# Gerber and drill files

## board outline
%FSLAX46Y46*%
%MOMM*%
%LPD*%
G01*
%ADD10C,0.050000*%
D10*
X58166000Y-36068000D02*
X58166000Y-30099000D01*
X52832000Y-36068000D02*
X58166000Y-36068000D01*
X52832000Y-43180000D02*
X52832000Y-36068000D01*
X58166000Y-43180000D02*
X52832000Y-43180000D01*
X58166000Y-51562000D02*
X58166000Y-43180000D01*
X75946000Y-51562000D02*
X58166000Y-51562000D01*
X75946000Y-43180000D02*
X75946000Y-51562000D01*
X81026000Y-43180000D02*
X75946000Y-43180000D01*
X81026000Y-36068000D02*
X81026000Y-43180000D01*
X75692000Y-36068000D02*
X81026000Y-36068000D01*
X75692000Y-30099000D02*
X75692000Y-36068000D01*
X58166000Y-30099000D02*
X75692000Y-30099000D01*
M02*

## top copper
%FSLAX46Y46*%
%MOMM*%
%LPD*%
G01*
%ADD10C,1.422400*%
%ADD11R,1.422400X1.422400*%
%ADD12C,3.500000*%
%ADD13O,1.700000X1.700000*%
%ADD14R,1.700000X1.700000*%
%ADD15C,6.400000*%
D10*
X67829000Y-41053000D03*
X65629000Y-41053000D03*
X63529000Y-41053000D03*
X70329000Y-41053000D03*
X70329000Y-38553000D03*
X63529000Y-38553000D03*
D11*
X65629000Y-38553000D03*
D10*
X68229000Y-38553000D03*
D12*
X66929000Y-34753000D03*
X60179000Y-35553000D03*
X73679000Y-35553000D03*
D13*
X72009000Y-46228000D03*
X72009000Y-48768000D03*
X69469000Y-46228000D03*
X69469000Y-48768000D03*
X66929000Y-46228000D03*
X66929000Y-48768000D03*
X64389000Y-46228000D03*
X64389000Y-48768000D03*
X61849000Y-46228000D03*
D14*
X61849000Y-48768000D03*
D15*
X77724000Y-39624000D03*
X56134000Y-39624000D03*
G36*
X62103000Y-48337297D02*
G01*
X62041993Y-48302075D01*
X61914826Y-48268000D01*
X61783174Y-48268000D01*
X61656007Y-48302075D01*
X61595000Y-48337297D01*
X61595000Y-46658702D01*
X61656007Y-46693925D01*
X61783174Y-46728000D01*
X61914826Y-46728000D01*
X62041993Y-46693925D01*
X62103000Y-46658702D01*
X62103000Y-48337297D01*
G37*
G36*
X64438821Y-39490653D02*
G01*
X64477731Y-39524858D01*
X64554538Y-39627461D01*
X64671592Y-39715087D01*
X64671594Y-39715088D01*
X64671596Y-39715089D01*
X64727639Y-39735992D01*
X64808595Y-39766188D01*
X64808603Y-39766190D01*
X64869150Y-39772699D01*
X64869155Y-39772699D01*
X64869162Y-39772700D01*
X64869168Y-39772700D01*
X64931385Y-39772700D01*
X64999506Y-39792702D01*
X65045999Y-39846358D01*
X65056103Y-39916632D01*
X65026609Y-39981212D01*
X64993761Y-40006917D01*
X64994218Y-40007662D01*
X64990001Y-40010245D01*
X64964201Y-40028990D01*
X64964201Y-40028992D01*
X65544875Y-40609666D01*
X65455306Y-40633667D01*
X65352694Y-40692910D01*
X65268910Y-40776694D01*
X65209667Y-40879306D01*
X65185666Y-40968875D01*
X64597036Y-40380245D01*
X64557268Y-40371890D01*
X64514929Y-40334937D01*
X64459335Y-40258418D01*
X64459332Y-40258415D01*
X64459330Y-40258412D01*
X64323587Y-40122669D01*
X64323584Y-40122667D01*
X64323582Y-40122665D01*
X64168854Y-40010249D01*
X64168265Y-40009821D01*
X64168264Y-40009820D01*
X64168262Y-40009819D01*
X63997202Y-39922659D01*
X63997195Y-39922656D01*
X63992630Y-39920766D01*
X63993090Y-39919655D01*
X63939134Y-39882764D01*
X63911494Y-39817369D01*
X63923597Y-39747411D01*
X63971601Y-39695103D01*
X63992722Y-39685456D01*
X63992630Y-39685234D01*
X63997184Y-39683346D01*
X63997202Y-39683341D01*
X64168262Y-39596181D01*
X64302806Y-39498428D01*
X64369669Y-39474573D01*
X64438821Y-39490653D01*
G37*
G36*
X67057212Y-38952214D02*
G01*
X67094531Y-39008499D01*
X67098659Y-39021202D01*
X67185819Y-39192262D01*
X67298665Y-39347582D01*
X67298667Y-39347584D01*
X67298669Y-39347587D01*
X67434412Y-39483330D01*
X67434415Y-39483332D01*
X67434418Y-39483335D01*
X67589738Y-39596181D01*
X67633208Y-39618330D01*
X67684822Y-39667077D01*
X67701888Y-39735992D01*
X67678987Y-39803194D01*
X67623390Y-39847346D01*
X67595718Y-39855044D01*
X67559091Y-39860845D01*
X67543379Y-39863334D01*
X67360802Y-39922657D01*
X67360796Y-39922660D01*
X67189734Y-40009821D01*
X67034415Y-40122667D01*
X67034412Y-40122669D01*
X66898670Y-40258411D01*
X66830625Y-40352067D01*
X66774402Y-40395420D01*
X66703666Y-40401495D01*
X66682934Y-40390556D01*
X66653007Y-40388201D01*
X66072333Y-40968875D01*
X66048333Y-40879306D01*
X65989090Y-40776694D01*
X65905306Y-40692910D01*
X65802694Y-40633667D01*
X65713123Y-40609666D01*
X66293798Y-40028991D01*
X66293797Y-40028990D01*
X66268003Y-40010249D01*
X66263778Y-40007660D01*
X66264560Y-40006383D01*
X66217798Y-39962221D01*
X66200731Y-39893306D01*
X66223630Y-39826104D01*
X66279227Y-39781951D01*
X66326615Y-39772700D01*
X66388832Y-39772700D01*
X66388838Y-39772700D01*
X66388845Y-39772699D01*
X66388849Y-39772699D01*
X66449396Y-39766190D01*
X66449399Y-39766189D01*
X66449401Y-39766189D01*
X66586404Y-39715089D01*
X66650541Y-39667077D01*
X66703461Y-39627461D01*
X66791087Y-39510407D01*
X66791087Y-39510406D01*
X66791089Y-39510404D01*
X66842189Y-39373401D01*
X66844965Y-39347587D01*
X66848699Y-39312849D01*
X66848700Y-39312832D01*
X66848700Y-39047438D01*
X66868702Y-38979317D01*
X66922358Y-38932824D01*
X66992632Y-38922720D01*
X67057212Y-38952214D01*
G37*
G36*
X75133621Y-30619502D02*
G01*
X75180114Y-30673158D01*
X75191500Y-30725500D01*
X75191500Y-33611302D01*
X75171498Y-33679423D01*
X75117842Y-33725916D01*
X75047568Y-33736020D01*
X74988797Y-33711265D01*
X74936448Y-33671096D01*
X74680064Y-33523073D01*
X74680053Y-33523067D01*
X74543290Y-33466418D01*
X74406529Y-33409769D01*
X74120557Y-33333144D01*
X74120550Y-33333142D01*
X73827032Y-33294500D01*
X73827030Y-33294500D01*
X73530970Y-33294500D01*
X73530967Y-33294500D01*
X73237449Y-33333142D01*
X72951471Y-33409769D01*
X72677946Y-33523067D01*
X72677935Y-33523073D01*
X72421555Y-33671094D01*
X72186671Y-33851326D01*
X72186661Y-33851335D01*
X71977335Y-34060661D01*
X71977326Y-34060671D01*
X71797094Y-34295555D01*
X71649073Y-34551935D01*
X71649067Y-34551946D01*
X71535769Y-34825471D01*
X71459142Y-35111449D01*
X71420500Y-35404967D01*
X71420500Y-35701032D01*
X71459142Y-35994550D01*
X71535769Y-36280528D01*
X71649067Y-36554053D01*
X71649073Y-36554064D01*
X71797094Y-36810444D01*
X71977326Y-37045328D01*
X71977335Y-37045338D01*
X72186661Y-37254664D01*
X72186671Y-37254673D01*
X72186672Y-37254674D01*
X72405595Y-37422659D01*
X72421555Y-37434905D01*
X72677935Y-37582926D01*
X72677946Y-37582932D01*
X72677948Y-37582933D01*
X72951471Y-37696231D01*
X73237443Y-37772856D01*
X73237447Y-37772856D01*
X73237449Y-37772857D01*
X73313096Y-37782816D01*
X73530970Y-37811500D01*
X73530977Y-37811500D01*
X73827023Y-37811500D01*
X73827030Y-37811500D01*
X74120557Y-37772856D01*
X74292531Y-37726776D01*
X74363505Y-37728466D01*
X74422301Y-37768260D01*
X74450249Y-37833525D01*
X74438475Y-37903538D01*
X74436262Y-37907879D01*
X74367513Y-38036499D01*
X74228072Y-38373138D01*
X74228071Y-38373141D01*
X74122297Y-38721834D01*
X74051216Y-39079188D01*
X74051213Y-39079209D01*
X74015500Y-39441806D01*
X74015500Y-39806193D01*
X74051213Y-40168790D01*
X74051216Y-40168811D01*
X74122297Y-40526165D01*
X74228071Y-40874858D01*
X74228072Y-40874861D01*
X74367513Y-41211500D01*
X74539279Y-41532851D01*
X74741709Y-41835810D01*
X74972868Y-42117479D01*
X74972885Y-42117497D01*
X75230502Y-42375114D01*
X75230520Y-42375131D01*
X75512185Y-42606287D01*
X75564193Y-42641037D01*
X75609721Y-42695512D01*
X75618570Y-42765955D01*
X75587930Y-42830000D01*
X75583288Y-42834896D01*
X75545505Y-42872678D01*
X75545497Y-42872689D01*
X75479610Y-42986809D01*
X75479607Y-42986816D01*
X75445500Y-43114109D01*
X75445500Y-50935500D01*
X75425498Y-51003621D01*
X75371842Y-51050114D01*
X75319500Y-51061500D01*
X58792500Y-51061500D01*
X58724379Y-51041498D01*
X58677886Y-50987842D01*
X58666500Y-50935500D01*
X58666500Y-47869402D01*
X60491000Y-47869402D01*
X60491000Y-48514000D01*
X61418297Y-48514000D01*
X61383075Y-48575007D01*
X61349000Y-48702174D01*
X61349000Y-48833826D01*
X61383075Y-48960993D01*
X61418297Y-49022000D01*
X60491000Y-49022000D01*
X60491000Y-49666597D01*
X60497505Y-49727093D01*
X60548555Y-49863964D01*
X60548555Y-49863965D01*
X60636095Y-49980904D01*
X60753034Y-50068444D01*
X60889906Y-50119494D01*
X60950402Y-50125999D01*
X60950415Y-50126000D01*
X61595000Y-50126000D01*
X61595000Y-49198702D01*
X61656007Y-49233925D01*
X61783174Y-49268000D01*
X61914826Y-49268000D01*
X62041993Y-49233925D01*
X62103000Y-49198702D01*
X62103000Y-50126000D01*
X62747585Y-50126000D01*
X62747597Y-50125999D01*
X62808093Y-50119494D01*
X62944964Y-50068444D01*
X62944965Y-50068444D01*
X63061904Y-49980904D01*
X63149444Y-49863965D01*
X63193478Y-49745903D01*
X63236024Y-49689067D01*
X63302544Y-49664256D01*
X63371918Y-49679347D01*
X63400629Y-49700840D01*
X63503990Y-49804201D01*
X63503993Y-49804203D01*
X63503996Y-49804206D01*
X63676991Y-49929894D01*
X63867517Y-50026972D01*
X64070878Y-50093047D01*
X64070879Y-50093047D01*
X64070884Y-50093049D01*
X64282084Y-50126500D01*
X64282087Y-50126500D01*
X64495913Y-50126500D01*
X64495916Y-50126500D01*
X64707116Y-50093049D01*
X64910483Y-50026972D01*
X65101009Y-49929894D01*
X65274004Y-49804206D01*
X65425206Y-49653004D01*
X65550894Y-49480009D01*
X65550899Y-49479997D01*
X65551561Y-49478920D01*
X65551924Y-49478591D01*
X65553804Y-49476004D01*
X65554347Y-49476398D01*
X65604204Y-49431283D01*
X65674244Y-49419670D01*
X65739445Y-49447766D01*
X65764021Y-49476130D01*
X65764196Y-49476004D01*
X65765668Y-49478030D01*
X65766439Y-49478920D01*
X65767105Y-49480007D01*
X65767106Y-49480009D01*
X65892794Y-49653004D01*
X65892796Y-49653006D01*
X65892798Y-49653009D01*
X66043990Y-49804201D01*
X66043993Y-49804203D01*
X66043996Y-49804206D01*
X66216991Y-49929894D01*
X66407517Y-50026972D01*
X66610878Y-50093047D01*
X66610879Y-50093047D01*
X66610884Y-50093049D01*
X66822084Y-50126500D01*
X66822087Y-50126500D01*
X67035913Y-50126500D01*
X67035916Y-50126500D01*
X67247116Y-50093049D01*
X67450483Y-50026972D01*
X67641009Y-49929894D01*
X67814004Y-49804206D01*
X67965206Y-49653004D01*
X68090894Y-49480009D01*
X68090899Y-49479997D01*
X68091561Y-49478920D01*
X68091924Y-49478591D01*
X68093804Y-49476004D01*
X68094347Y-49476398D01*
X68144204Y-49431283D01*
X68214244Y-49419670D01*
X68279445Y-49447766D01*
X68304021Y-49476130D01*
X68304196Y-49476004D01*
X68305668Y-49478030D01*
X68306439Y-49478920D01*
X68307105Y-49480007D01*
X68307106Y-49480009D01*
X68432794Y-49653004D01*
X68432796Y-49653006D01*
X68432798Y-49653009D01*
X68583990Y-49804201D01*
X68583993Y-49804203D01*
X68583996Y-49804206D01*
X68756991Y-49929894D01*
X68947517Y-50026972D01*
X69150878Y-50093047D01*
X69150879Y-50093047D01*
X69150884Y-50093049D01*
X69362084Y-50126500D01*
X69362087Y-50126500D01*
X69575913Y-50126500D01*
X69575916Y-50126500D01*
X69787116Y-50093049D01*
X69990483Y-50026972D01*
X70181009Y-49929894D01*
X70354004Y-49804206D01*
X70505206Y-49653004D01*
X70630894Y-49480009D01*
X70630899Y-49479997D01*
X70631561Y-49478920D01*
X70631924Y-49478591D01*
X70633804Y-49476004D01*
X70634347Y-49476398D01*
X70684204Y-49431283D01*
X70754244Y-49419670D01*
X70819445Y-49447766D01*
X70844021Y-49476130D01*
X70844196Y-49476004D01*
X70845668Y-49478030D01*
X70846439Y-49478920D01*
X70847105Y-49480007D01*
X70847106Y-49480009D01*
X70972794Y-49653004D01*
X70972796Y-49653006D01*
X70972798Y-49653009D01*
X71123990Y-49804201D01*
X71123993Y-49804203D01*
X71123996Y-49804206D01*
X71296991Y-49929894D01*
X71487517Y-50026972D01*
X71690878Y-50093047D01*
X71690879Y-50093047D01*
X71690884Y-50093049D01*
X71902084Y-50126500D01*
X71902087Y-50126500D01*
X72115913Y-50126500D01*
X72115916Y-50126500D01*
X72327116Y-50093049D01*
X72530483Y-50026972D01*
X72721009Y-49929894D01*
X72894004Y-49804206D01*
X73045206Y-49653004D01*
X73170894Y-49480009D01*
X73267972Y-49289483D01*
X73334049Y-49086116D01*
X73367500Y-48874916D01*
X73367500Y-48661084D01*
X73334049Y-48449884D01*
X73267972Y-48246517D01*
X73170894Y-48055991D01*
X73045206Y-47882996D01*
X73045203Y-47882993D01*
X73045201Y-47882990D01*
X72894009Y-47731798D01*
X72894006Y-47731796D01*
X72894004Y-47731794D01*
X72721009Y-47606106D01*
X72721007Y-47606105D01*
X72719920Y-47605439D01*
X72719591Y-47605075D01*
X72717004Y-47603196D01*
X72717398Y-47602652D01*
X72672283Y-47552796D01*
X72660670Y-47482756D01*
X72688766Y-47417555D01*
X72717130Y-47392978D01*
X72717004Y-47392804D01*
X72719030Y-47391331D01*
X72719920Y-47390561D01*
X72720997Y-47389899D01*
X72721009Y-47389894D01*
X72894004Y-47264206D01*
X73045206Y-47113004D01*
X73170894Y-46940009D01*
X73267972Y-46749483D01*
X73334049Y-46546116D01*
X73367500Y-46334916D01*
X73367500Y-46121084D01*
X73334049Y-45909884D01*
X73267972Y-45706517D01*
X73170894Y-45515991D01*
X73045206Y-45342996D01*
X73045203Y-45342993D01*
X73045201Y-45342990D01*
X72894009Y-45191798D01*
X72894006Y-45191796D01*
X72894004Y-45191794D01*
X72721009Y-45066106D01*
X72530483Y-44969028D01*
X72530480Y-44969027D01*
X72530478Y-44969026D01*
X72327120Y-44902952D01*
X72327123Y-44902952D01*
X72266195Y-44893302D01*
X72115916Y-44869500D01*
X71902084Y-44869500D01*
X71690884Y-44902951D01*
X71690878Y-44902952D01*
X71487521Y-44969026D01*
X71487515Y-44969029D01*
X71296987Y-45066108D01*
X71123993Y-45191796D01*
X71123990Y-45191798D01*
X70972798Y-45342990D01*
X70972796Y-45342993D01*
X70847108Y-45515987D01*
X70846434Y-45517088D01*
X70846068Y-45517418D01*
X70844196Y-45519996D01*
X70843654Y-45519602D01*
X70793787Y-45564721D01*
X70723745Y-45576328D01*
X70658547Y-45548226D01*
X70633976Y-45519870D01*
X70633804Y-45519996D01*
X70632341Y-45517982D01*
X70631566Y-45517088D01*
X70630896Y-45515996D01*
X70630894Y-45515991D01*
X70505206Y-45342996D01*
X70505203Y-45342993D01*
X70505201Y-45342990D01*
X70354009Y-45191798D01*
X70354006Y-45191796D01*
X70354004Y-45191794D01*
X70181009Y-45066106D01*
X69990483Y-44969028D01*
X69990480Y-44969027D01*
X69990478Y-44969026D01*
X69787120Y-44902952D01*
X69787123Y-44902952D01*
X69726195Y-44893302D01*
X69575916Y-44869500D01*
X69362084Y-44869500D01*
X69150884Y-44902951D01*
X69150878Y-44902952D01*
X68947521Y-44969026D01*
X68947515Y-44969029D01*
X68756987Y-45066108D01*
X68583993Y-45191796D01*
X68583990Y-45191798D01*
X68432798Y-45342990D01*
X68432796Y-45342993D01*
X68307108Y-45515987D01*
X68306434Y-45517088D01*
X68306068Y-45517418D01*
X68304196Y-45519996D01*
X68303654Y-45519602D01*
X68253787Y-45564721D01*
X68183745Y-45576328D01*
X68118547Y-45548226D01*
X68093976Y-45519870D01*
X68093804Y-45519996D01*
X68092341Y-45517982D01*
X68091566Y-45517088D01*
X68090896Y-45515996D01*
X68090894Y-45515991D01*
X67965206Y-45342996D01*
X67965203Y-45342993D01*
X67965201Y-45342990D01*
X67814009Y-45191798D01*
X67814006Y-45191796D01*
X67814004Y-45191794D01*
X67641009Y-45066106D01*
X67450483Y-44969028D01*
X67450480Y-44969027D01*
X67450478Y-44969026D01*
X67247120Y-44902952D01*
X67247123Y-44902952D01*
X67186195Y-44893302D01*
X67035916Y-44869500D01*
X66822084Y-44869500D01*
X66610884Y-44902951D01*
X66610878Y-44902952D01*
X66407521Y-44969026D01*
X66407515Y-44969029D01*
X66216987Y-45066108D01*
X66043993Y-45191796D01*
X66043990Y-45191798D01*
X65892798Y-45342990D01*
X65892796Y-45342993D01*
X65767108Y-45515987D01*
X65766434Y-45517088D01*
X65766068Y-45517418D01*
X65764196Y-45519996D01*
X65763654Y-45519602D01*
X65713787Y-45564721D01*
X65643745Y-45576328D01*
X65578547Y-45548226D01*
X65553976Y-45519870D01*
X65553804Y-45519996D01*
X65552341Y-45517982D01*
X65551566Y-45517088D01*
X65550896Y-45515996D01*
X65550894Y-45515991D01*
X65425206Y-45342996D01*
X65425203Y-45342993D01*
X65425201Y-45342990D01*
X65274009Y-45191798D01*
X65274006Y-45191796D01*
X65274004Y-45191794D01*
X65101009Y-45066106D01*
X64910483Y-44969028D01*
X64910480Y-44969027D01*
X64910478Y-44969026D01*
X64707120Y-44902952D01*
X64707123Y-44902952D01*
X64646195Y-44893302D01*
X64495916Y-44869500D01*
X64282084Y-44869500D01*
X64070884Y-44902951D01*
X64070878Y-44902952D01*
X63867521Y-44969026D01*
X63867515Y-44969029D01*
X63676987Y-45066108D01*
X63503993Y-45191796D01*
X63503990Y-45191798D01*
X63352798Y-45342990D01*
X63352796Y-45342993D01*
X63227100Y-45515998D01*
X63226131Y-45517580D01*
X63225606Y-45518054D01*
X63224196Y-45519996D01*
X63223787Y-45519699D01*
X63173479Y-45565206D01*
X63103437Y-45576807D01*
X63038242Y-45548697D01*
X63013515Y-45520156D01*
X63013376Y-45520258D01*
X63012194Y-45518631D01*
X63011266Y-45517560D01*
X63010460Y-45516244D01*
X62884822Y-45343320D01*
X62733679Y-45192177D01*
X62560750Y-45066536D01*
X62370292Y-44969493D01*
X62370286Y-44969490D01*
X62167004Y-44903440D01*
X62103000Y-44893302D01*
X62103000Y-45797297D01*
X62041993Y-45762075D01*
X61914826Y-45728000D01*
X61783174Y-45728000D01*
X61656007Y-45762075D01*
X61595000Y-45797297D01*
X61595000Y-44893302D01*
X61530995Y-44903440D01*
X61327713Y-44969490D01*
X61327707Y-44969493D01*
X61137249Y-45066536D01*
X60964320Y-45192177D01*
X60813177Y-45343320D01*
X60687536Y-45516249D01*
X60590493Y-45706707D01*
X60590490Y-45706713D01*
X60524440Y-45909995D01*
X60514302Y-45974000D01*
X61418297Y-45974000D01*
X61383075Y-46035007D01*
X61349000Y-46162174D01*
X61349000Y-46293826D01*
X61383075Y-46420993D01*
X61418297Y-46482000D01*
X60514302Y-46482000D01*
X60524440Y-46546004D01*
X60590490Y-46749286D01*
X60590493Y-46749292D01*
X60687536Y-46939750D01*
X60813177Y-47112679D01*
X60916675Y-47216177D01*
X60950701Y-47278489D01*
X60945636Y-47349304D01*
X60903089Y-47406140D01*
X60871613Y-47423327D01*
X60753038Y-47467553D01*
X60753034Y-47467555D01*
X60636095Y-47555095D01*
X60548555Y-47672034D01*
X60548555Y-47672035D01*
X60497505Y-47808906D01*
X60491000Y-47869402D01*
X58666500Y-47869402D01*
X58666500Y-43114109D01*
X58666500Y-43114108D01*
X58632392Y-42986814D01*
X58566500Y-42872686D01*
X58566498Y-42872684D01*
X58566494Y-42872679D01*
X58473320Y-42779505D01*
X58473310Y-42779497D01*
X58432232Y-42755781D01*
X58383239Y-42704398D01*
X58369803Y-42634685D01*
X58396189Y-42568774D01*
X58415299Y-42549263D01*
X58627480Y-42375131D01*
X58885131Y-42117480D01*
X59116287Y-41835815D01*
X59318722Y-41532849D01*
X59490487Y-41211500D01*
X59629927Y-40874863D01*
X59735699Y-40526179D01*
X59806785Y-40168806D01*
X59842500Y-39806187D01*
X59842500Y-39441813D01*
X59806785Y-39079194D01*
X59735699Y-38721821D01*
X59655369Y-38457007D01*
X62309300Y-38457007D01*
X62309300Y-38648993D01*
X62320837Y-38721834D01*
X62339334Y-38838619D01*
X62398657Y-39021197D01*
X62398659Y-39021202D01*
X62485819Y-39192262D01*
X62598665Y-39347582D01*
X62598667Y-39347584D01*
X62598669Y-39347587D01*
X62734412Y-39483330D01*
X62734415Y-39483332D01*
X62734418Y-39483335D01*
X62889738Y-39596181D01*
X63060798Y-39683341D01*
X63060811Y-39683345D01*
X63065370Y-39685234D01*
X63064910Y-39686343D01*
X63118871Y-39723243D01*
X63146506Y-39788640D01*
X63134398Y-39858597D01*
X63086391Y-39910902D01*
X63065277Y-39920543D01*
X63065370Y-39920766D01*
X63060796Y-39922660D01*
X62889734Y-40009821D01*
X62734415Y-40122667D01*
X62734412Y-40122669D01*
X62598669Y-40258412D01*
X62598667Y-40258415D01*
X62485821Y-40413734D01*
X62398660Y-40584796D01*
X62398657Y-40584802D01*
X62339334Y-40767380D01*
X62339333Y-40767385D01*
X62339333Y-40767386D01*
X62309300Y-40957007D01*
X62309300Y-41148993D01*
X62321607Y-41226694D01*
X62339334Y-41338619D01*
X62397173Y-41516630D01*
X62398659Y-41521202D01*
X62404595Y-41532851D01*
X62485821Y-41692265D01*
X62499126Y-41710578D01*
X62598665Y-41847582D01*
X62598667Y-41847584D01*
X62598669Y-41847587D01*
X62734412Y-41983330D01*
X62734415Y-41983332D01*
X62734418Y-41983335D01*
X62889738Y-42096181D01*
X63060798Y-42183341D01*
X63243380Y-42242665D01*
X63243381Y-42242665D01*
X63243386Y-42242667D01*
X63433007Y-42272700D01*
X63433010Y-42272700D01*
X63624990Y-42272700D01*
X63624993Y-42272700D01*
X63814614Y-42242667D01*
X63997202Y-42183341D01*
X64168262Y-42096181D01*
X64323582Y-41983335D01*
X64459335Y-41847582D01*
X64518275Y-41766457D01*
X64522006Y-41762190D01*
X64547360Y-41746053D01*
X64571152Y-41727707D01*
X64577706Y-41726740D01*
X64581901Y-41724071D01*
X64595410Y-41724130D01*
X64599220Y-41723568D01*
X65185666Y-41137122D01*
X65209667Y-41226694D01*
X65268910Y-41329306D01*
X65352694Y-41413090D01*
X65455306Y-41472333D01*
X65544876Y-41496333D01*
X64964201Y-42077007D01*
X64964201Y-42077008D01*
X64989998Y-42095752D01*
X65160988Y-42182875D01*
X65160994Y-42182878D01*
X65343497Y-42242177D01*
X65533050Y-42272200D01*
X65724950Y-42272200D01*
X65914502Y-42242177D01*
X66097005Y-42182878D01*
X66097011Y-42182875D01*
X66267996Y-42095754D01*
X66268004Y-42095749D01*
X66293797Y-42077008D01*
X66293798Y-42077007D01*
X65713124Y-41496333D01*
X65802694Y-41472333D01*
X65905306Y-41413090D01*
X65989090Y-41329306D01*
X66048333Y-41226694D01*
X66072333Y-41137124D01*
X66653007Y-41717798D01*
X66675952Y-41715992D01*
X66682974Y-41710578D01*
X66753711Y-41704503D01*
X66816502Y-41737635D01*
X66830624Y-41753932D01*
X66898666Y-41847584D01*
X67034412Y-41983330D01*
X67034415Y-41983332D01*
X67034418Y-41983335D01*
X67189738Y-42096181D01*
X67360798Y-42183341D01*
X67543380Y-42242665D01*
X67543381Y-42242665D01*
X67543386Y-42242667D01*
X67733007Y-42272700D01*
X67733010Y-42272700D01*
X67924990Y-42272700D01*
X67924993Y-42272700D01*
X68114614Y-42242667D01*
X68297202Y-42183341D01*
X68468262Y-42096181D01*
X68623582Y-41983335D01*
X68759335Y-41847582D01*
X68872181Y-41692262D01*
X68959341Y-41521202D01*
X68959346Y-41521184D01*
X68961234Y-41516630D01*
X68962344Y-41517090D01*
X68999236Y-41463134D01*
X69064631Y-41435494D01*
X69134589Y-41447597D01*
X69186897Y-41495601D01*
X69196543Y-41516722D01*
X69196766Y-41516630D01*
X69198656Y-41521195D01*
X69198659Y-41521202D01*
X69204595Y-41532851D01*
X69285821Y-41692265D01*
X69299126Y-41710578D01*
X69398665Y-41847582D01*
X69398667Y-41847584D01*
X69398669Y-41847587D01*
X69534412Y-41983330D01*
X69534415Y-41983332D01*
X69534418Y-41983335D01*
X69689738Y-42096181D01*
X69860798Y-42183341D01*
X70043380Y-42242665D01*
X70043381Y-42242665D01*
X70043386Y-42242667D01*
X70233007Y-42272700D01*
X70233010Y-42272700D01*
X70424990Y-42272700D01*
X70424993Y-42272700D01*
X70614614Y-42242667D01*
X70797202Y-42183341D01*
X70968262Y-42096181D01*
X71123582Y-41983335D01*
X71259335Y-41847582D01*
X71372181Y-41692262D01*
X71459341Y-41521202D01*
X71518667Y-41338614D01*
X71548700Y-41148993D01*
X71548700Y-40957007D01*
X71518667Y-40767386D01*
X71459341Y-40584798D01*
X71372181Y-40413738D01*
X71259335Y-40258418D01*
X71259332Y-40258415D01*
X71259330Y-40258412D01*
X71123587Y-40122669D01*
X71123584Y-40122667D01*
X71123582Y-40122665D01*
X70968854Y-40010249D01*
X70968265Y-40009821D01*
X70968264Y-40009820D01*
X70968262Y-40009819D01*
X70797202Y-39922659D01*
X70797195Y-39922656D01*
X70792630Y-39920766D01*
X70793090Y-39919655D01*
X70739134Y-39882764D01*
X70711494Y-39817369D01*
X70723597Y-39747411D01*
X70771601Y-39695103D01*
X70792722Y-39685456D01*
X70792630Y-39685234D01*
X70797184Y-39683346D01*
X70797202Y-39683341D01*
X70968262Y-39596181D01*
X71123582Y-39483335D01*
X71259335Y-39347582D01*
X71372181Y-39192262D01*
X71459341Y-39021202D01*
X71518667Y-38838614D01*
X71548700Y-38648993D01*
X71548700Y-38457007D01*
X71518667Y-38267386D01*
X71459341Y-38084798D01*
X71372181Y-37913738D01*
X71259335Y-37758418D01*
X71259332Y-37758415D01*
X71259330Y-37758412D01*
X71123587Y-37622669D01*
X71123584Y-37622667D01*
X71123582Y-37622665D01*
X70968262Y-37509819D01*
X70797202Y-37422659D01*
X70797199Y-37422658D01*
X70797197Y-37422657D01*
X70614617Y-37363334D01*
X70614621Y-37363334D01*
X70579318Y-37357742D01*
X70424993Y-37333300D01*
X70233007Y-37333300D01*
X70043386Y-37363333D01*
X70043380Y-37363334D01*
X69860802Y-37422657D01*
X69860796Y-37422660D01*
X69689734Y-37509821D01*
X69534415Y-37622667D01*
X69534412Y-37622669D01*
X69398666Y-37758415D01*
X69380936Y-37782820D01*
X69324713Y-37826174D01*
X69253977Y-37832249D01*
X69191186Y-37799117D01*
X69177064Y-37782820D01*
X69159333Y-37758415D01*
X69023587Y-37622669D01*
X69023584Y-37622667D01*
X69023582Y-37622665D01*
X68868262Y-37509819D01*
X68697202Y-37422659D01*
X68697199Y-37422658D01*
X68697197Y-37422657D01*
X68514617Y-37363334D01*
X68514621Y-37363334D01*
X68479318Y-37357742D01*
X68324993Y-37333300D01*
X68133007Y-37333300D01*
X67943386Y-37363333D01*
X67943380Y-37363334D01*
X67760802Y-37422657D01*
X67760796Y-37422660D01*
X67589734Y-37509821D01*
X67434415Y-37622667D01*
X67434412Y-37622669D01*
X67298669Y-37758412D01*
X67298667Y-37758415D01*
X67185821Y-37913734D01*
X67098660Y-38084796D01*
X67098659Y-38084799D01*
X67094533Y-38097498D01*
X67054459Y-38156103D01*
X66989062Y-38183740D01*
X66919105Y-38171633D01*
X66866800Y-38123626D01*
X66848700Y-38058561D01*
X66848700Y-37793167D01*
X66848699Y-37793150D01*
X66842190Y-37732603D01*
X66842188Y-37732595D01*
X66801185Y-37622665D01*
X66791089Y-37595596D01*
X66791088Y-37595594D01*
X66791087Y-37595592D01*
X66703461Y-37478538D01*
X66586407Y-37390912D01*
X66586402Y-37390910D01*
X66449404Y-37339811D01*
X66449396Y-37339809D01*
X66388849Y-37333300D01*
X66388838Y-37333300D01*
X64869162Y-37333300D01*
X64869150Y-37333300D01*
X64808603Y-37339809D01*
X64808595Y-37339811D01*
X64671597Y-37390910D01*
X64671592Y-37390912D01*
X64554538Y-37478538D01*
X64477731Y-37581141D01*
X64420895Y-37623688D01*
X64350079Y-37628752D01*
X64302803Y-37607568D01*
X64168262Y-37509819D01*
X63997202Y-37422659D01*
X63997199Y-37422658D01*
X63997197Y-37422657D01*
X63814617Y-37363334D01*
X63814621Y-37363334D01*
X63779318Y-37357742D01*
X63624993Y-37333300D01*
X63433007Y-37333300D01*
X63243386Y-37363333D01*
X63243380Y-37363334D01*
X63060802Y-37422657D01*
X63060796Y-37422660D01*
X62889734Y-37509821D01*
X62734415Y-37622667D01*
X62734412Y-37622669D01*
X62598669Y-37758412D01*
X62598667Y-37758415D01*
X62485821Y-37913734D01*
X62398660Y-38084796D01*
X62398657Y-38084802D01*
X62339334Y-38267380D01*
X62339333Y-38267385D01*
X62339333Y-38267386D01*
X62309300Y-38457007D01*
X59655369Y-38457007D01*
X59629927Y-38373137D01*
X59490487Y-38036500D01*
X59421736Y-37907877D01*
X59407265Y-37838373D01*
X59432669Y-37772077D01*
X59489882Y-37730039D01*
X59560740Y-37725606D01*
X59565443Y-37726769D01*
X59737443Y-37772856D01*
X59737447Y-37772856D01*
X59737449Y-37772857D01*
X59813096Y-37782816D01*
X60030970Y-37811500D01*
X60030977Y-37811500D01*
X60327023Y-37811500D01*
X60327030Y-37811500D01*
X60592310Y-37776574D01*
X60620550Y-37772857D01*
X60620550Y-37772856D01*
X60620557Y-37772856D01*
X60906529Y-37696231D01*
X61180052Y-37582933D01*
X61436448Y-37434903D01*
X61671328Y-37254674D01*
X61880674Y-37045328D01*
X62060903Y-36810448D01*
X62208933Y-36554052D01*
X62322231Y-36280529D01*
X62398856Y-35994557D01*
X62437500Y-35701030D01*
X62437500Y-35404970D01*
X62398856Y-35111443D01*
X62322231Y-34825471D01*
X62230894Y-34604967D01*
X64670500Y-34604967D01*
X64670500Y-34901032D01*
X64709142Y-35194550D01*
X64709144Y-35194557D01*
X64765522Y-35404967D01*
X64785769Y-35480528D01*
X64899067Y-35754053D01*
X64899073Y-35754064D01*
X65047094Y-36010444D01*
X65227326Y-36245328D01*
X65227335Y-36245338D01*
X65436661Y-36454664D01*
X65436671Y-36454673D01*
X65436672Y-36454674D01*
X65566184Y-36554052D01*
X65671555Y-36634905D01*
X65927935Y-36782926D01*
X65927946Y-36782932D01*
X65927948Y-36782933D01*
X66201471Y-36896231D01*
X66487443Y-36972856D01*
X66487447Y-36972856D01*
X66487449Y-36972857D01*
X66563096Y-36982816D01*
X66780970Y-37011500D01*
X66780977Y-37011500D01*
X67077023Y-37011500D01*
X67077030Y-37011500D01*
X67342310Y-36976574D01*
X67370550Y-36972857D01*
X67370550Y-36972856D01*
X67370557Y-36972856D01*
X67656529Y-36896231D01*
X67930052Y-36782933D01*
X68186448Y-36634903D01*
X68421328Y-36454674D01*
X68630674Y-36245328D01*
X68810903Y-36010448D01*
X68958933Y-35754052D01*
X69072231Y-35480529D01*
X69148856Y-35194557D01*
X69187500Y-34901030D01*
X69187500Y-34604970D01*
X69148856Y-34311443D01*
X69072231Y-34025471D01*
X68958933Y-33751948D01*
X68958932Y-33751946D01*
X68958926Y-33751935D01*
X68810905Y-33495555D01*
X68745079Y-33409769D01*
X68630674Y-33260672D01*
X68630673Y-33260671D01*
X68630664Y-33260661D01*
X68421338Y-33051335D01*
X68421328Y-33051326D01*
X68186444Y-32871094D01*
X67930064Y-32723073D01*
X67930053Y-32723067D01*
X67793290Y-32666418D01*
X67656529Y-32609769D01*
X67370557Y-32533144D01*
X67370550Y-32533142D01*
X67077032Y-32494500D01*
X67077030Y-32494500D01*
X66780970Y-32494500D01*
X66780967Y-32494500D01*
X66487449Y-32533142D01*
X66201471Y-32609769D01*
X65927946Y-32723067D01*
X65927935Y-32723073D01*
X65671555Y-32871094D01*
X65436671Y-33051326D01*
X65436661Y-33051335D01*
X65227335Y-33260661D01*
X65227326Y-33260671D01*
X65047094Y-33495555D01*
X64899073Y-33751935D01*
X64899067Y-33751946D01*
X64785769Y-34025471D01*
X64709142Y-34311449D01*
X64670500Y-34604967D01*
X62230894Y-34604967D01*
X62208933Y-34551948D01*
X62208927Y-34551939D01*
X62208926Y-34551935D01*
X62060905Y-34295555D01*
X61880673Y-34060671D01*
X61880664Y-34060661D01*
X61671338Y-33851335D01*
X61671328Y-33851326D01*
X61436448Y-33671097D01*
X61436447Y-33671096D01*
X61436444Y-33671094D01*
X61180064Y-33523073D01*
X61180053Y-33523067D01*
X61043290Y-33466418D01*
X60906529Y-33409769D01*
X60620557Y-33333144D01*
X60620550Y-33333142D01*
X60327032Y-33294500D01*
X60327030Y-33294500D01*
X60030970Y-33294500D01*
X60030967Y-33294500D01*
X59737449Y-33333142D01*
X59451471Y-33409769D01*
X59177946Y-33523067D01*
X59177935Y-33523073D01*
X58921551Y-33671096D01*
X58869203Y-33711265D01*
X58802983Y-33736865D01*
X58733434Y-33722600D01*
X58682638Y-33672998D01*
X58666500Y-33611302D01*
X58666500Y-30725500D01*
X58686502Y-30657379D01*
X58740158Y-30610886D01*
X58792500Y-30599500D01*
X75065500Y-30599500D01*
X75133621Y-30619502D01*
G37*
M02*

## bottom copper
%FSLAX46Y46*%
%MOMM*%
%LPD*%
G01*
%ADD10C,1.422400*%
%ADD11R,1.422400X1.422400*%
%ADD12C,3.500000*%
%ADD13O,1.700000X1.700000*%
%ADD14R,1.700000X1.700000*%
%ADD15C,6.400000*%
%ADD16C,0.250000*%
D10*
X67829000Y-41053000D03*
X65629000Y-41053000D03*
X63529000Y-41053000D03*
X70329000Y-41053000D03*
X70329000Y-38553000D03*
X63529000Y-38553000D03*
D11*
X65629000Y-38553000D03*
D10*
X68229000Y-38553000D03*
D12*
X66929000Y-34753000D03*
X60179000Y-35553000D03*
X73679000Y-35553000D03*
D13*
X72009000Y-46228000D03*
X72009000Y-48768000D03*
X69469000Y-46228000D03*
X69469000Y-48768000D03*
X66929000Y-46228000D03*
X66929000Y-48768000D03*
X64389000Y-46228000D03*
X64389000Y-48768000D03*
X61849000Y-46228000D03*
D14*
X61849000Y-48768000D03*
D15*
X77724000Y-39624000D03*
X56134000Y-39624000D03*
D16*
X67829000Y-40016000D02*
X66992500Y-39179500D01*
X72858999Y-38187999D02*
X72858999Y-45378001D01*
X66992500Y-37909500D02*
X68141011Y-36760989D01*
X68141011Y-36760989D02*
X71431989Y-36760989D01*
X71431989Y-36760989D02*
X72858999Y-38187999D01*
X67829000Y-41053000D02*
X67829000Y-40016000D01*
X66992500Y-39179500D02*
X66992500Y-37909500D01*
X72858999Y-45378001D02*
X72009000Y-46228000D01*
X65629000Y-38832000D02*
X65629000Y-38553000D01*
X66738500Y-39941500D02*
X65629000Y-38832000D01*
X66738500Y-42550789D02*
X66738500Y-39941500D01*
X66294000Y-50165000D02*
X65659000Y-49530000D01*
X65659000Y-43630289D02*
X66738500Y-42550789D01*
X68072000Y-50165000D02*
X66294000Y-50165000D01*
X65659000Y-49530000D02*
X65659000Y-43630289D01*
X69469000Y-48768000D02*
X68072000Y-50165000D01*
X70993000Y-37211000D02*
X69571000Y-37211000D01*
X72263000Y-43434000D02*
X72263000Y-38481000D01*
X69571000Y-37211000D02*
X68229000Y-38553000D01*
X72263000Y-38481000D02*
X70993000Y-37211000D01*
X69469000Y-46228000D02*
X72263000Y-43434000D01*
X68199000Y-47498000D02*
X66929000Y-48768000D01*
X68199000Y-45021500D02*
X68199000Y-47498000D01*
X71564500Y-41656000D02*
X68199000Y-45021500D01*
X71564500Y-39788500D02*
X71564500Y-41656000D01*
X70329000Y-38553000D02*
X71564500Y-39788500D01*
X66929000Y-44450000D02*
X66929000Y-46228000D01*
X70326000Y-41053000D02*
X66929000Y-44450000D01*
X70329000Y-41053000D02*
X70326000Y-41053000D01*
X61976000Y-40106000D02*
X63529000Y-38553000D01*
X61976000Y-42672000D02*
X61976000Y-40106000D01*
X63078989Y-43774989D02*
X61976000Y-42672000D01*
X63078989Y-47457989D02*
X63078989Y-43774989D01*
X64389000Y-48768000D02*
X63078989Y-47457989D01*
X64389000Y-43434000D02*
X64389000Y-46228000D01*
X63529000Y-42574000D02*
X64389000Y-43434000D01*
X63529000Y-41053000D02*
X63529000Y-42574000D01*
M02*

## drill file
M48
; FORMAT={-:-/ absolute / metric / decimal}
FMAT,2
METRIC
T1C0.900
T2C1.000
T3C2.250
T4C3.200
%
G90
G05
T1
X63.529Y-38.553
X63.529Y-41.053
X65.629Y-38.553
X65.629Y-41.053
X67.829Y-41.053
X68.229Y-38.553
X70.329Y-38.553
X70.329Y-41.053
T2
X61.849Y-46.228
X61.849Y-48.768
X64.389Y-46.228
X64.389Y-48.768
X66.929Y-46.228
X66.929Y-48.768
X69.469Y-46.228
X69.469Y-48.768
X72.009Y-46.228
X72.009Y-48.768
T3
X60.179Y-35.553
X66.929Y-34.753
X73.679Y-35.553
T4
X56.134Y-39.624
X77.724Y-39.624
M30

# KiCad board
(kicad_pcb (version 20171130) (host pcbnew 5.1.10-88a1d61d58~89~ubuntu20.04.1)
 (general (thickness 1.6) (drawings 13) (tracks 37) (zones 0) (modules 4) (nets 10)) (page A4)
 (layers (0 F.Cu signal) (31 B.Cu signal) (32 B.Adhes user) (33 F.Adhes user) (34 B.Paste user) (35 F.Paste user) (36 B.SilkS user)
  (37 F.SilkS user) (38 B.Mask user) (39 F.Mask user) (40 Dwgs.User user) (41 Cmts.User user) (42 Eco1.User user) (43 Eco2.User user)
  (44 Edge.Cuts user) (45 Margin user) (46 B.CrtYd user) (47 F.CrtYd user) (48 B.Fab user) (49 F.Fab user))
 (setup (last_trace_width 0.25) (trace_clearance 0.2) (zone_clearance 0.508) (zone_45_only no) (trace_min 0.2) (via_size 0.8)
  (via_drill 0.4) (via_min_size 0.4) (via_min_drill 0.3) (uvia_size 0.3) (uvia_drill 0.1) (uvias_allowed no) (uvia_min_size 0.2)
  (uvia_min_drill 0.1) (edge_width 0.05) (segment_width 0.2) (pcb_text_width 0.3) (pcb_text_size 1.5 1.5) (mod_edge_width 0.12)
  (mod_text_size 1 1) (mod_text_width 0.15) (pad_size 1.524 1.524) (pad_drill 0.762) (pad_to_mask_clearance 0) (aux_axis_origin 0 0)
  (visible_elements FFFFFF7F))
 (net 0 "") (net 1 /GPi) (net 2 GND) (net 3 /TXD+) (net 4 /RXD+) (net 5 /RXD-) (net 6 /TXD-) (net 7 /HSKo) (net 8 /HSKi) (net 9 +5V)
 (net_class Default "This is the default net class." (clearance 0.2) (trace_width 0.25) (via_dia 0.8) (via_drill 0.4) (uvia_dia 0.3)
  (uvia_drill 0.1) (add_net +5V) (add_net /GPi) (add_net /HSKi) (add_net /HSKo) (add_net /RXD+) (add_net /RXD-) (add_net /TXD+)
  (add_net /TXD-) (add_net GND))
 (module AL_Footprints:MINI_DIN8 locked (layer F.Cu) (at 66.929 34.753)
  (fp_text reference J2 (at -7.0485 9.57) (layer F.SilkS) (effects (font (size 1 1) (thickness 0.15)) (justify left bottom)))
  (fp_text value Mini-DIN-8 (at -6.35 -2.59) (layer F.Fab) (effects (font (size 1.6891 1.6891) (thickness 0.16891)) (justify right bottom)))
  (pad 7 thru_hole circle (at 0.9 6.3) (size 1.4224 1.4224) (drill 0.9) (layers *.Cu *.Mask) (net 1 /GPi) (solder_mask_margin 0.0508))
  (pad 4 thru_hole circle (at -1.3 6.3) (size 1.4224 1.4224) (drill 0.9) (layers *.Cu *.Mask) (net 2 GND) (solder_mask_margin 0.0508))
  (pad 6 thru_hole circle (at -3.4 6.3) (size 1.4224 1.4224) (drill 0.9) (layers *.Cu *.Mask) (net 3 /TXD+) (solder_mask_margin 0.0508))
  (pad 8 thru_hole circle (at 3.4 6.3) (size 1.4224 1.4224) (drill 0.9) (layers *.Cu *.Mask) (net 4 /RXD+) (solder_mask_margin 0.0508))
  (pad 5 thru_hole circle (at 3.4 3.8) (size 1.4224 1.4224) (drill 0.9) (layers *.Cu *.Mask) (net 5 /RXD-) (solder_mask_margin 0.0508))
  (pad 3 thru_hole circle (at -3.4 3.8) (size 1.4224 1.4224) (drill 0.9) (layers *.Cu *.Mask) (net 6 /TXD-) (solder_mask_margin 0.0508))
  (pad 1 thru_hole rect (at -1.3 3.8) (size 1.4224 1.4224) (drill 0.9) (layers *.Cu *.Mask) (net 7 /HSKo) (solder_mask_margin 0.0508))
  (pad 2 thru_hole circle (at 1.3 3.8) (size 1.4224 1.4224) (drill 0.9) (layers *.Cu *.Mask) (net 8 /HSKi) (solder_mask_margin 0.0508))
  (pad SH2 thru_hole circle (at 0 0) (size 3.5 3.5) (drill 2.25) (layers *.Cu *.Mask) (solder_mask_margin 0.0508))
  (pad SH3 thru_hole circle (at -6.75 0.8) (size 3.5 3.5) (drill 2.25) (layers *.Cu *.Mask) (solder_mask_margin 0.0508))
  (pad SH1 thru_hole circle (at 6.75 0.8) (size 3.5 3.5) (drill 2.25) (layers *.Cu *.Mask) (solder_mask_margin 0.0508)))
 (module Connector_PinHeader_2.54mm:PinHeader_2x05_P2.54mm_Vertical (layer F.Cu) (at 61.849 48.768 90)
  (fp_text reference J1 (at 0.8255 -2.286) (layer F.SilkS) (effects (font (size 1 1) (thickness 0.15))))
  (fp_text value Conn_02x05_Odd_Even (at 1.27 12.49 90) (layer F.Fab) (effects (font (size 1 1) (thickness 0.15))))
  (pad 10 thru_hole oval (at 2.54 10.16 90) (size 1.7 1.7) (drill 1) (layers *.Cu *.Mask) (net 1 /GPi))
  (pad 9 thru_hole oval (at 0 10.16 90) (size 1.7 1.7) (drill 1) (layers *.Cu *.Mask) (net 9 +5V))
  (pad 8 thru_hole oval (at 2.54 7.62 90) (size 1.7 1.7) (drill 1) (layers *.Cu *.Mask) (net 8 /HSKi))
  (pad 7 thru_hole oval (at 0 7.62 90) (size 1.7 1.7) (drill 1) (layers *.Cu *.Mask) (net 7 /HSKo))
  (pad 6 thru_hole oval (at 2.54 5.08 90) (size 1.7 1.7) (drill 1) (layers *.Cu *.Mask) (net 4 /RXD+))
  (pad 5 thru_hole oval (at 0 5.08 90) (size 1.7 1.7) (drill 1) (layers *.Cu *.Mask) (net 5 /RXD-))
  (pad 4 thru_hole oval (at 2.54 2.54 90) (size 1.7 1.7) (drill 1) (layers *.Cu *.Mask) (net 3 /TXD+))
  (pad 3 thru_hole oval (at 0 2.54 90) (size 1.7 1.7) (drill 1) (layers *.Cu *.Mask) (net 6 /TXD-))
  (pad 2 thru_hole oval (at 2.54 0 90) (size 1.7 1.7) (drill 1) (layers *.Cu *.Mask) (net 2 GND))
  (pad 1 thru_hole rect (at 0 0 90) (size 1.7 1.7) (drill 1) (layers *.Cu *.Mask) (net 2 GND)))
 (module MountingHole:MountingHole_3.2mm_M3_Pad (layer F.Cu) (at 77.724 39.624)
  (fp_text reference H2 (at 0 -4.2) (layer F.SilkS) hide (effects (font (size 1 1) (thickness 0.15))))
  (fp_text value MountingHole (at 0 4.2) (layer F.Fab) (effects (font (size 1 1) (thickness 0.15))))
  (pad 1 thru_hole circle (at 0 0) (size 6.4 6.4) (drill 3.2) (layers *.Cu *.Mask)))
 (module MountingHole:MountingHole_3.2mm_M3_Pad (layer F.Cu) (at 56.134 39.624)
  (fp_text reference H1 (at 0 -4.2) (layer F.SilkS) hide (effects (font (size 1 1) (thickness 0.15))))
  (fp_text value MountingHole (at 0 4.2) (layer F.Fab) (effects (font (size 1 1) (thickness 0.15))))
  (pad 1 thru_hole circle (at 0 0) (size 6.4 6.4) (drill 3.2) (layers *.Cu *.Mask)))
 (gr_line (start 58.166 36.068) (end 58.166 30.099) (layer Edge.Cuts) (width 0.05))
 (gr_line (start 52.832 36.068) (end 58.166 36.068) (layer Edge.Cuts) (width 0.05))
 (gr_line (start 52.832 43.18) (end 52.832 36.068) (layer Edge.Cuts) (width 0.05))
 (gr_line (start 58.166 43.18) (end 52.832 43.18) (layer Edge.Cuts) (width 0.05))
 (gr_line (start 58.166 51.562) (end 58.166 43.18) (layer Edge.Cuts) (width 0.05))
 (gr_line (start 75.946 51.562) (end 58.166 51.562) (layer Edge.Cuts) (width 0.05))
 (gr_line (start 75.946 43.18) (end 75.946 51.562) (layer Edge.Cuts) (width 0.05))
 (gr_line (start 81.026 43.18) (end 75.946 43.18) (layer Edge.Cuts) (width 0.05))
 (gr_line (start 81.026 36.068) (end 81.026 43.18) (layer Edge.Cuts) (width 0.05))
 (gr_line (start 75.692 36.068) (end 81.026 36.068) (layer Edge.Cuts) (width 0.05))
 (gr_line (start 75.692 30.099) (end 75.692 36.068) (layer Edge.Cuts) (width 0.05))
 (gr_line (start 58.166 30.099) (end 75.692 30.099) (layer Edge.Cuts) (width 0.05))
 (segment (start 67.829 40.016) (end 66.9925 39.1795) (width 0.25) (layer B.Cu) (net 1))
 (segment (start 72.858999 38.187999) (end 72.858999 45.378001) (width 0.25) (layer B.Cu) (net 1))
 (segment (start 66.9925 37.9095) (end 68.141011 36.760989) (width 0.25) (layer B.Cu) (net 1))
 (segment (start 68.141011 36.760989) (end 71.431989 36.760989) (width 0.25) (layer B.Cu) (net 1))
 (segment (start 71.431989 36.760989) (end 72.858999 38.187999) (width 0.25) (layer B.Cu) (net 1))
 (segment (start 67.829 41.053) (end 67.829 40.016) (width 0.25) (layer B.Cu) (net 1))
 (segment (start 66.9925 39.1795) (end 66.9925 37.9095) (width 0.25) (layer B.Cu) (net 1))
 (segment (start 72.858999 45.378001) (end 72.009 46.228) (width 0.25) (layer B.Cu) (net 1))
 (segment (start 65.629 38.832) (end 65.629 38.553) (width 0.25) (layer B.Cu) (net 7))
 (segment (start 66.7385 39.9415) (end 65.629 38.832) (width 0.25) (layer B.Cu) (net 7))
 (segment (start 66.7385 42.550789) (end 66.7385 39.9415) (width 0.25) (layer B.Cu) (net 7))
 (segment (start 66.294 50.165) (end 65.659 49.53) (width 0.25) (layer B.Cu) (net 7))
 (segment (start 65.659 43.630289) (end 66.7385 42.550789) (width 0.25) (layer B.Cu) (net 7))
 (segment (start 68.072 50.165) (end 66.294 50.165) (width 0.25) (layer B.Cu) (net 7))
 (segment (start 65.659 49.53) (end 65.659 43.630289) (width 0.25) (layer B.Cu) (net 7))
 (segment (start 69.469 48.768) (end 68.072 50.165) (width 0.25) (layer B.Cu) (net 7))
 (segment (start 70.993 37.211) (end 69.571 37.211) (width 0.25) (layer B.Cu) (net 8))
 (segment (start 72.263 43.434) (end 72.263 38.481) (width 0.25) (layer B.Cu) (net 8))
 (segment (start 69.571 37.211) (end 68.229 38.553) (width 0.25) (layer B.Cu) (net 8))
 (segment (start 72.263 38.481) (end 70.993 37.211) (width 0.25) (layer B.Cu) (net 8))
 (segment (start 69.469 46.228) (end 72.263 43.434) (width 0.25) (layer B.Cu) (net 8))
 (segment (start 68.199 47.498) (end 66.929 48.768) (width 0.25) (layer B.Cu) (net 5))
 (segment (start 68.199 45.0215) (end 68.199 47.498) (width 0.25) (layer B.Cu) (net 5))
 (segment (start 71.5645 41.656) (end 68.199 45.0215) (width 0.25) (layer B.Cu) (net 5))
 (segment (start 71.5645 39.7885) (end 71.5645 41.656) (width 0.25) (layer B.Cu) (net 5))
 (segment (start 70.329 38.553) (end 71.5645 39.7885) (width 0.25) (layer B.Cu) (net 5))
 (segment (start 66.929 44.45) (end 66.929 46.228) (width 0.25) (layer B.Cu) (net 4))
 (segment (start 70.326 41.053) (end 66.929 44.45) (width 0.25) (layer B.Cu) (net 4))
 (segment (start 70.329 41.053) (end 70.326 41.053) (width 0.25) (layer B.Cu) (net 4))
 (segment (start 61.976 40.106) (end 63.529 38.553) (width 0.25) (layer B.Cu) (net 6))
 (segment (start 61.976 42.672) (end 61.976 40.106) (width 0.25) (layer B.Cu) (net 6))
 (segment (start 63.078989 43.774989) (end 61.976 42.672) (width 0.25) (layer B.Cu) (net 6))
 (segment (start 63.078989 47.457989) (end 63.078989 43.774989) (width 0.25) (layer B.Cu) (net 6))
 (segment (start 64.389 48.768) (end 63.078989 47.457989) (width 0.25) (layer B.Cu) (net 6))
 (segment (start 64.389 43.434) (end 64.389 46.228) (width 0.25) (layer B.Cu) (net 3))
 (segment (start 63.529 42.574) (end 64.389 43.434) (width 0.25) (layer B.Cu) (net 3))
 (segment (start 63.529 41.053) (end 63.529 42.574) (width 0.25) (layer B.Cu) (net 3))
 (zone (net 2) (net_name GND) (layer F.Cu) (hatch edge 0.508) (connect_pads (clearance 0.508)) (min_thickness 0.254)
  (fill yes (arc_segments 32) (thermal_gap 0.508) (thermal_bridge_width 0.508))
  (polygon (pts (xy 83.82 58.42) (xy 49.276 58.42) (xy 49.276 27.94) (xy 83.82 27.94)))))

